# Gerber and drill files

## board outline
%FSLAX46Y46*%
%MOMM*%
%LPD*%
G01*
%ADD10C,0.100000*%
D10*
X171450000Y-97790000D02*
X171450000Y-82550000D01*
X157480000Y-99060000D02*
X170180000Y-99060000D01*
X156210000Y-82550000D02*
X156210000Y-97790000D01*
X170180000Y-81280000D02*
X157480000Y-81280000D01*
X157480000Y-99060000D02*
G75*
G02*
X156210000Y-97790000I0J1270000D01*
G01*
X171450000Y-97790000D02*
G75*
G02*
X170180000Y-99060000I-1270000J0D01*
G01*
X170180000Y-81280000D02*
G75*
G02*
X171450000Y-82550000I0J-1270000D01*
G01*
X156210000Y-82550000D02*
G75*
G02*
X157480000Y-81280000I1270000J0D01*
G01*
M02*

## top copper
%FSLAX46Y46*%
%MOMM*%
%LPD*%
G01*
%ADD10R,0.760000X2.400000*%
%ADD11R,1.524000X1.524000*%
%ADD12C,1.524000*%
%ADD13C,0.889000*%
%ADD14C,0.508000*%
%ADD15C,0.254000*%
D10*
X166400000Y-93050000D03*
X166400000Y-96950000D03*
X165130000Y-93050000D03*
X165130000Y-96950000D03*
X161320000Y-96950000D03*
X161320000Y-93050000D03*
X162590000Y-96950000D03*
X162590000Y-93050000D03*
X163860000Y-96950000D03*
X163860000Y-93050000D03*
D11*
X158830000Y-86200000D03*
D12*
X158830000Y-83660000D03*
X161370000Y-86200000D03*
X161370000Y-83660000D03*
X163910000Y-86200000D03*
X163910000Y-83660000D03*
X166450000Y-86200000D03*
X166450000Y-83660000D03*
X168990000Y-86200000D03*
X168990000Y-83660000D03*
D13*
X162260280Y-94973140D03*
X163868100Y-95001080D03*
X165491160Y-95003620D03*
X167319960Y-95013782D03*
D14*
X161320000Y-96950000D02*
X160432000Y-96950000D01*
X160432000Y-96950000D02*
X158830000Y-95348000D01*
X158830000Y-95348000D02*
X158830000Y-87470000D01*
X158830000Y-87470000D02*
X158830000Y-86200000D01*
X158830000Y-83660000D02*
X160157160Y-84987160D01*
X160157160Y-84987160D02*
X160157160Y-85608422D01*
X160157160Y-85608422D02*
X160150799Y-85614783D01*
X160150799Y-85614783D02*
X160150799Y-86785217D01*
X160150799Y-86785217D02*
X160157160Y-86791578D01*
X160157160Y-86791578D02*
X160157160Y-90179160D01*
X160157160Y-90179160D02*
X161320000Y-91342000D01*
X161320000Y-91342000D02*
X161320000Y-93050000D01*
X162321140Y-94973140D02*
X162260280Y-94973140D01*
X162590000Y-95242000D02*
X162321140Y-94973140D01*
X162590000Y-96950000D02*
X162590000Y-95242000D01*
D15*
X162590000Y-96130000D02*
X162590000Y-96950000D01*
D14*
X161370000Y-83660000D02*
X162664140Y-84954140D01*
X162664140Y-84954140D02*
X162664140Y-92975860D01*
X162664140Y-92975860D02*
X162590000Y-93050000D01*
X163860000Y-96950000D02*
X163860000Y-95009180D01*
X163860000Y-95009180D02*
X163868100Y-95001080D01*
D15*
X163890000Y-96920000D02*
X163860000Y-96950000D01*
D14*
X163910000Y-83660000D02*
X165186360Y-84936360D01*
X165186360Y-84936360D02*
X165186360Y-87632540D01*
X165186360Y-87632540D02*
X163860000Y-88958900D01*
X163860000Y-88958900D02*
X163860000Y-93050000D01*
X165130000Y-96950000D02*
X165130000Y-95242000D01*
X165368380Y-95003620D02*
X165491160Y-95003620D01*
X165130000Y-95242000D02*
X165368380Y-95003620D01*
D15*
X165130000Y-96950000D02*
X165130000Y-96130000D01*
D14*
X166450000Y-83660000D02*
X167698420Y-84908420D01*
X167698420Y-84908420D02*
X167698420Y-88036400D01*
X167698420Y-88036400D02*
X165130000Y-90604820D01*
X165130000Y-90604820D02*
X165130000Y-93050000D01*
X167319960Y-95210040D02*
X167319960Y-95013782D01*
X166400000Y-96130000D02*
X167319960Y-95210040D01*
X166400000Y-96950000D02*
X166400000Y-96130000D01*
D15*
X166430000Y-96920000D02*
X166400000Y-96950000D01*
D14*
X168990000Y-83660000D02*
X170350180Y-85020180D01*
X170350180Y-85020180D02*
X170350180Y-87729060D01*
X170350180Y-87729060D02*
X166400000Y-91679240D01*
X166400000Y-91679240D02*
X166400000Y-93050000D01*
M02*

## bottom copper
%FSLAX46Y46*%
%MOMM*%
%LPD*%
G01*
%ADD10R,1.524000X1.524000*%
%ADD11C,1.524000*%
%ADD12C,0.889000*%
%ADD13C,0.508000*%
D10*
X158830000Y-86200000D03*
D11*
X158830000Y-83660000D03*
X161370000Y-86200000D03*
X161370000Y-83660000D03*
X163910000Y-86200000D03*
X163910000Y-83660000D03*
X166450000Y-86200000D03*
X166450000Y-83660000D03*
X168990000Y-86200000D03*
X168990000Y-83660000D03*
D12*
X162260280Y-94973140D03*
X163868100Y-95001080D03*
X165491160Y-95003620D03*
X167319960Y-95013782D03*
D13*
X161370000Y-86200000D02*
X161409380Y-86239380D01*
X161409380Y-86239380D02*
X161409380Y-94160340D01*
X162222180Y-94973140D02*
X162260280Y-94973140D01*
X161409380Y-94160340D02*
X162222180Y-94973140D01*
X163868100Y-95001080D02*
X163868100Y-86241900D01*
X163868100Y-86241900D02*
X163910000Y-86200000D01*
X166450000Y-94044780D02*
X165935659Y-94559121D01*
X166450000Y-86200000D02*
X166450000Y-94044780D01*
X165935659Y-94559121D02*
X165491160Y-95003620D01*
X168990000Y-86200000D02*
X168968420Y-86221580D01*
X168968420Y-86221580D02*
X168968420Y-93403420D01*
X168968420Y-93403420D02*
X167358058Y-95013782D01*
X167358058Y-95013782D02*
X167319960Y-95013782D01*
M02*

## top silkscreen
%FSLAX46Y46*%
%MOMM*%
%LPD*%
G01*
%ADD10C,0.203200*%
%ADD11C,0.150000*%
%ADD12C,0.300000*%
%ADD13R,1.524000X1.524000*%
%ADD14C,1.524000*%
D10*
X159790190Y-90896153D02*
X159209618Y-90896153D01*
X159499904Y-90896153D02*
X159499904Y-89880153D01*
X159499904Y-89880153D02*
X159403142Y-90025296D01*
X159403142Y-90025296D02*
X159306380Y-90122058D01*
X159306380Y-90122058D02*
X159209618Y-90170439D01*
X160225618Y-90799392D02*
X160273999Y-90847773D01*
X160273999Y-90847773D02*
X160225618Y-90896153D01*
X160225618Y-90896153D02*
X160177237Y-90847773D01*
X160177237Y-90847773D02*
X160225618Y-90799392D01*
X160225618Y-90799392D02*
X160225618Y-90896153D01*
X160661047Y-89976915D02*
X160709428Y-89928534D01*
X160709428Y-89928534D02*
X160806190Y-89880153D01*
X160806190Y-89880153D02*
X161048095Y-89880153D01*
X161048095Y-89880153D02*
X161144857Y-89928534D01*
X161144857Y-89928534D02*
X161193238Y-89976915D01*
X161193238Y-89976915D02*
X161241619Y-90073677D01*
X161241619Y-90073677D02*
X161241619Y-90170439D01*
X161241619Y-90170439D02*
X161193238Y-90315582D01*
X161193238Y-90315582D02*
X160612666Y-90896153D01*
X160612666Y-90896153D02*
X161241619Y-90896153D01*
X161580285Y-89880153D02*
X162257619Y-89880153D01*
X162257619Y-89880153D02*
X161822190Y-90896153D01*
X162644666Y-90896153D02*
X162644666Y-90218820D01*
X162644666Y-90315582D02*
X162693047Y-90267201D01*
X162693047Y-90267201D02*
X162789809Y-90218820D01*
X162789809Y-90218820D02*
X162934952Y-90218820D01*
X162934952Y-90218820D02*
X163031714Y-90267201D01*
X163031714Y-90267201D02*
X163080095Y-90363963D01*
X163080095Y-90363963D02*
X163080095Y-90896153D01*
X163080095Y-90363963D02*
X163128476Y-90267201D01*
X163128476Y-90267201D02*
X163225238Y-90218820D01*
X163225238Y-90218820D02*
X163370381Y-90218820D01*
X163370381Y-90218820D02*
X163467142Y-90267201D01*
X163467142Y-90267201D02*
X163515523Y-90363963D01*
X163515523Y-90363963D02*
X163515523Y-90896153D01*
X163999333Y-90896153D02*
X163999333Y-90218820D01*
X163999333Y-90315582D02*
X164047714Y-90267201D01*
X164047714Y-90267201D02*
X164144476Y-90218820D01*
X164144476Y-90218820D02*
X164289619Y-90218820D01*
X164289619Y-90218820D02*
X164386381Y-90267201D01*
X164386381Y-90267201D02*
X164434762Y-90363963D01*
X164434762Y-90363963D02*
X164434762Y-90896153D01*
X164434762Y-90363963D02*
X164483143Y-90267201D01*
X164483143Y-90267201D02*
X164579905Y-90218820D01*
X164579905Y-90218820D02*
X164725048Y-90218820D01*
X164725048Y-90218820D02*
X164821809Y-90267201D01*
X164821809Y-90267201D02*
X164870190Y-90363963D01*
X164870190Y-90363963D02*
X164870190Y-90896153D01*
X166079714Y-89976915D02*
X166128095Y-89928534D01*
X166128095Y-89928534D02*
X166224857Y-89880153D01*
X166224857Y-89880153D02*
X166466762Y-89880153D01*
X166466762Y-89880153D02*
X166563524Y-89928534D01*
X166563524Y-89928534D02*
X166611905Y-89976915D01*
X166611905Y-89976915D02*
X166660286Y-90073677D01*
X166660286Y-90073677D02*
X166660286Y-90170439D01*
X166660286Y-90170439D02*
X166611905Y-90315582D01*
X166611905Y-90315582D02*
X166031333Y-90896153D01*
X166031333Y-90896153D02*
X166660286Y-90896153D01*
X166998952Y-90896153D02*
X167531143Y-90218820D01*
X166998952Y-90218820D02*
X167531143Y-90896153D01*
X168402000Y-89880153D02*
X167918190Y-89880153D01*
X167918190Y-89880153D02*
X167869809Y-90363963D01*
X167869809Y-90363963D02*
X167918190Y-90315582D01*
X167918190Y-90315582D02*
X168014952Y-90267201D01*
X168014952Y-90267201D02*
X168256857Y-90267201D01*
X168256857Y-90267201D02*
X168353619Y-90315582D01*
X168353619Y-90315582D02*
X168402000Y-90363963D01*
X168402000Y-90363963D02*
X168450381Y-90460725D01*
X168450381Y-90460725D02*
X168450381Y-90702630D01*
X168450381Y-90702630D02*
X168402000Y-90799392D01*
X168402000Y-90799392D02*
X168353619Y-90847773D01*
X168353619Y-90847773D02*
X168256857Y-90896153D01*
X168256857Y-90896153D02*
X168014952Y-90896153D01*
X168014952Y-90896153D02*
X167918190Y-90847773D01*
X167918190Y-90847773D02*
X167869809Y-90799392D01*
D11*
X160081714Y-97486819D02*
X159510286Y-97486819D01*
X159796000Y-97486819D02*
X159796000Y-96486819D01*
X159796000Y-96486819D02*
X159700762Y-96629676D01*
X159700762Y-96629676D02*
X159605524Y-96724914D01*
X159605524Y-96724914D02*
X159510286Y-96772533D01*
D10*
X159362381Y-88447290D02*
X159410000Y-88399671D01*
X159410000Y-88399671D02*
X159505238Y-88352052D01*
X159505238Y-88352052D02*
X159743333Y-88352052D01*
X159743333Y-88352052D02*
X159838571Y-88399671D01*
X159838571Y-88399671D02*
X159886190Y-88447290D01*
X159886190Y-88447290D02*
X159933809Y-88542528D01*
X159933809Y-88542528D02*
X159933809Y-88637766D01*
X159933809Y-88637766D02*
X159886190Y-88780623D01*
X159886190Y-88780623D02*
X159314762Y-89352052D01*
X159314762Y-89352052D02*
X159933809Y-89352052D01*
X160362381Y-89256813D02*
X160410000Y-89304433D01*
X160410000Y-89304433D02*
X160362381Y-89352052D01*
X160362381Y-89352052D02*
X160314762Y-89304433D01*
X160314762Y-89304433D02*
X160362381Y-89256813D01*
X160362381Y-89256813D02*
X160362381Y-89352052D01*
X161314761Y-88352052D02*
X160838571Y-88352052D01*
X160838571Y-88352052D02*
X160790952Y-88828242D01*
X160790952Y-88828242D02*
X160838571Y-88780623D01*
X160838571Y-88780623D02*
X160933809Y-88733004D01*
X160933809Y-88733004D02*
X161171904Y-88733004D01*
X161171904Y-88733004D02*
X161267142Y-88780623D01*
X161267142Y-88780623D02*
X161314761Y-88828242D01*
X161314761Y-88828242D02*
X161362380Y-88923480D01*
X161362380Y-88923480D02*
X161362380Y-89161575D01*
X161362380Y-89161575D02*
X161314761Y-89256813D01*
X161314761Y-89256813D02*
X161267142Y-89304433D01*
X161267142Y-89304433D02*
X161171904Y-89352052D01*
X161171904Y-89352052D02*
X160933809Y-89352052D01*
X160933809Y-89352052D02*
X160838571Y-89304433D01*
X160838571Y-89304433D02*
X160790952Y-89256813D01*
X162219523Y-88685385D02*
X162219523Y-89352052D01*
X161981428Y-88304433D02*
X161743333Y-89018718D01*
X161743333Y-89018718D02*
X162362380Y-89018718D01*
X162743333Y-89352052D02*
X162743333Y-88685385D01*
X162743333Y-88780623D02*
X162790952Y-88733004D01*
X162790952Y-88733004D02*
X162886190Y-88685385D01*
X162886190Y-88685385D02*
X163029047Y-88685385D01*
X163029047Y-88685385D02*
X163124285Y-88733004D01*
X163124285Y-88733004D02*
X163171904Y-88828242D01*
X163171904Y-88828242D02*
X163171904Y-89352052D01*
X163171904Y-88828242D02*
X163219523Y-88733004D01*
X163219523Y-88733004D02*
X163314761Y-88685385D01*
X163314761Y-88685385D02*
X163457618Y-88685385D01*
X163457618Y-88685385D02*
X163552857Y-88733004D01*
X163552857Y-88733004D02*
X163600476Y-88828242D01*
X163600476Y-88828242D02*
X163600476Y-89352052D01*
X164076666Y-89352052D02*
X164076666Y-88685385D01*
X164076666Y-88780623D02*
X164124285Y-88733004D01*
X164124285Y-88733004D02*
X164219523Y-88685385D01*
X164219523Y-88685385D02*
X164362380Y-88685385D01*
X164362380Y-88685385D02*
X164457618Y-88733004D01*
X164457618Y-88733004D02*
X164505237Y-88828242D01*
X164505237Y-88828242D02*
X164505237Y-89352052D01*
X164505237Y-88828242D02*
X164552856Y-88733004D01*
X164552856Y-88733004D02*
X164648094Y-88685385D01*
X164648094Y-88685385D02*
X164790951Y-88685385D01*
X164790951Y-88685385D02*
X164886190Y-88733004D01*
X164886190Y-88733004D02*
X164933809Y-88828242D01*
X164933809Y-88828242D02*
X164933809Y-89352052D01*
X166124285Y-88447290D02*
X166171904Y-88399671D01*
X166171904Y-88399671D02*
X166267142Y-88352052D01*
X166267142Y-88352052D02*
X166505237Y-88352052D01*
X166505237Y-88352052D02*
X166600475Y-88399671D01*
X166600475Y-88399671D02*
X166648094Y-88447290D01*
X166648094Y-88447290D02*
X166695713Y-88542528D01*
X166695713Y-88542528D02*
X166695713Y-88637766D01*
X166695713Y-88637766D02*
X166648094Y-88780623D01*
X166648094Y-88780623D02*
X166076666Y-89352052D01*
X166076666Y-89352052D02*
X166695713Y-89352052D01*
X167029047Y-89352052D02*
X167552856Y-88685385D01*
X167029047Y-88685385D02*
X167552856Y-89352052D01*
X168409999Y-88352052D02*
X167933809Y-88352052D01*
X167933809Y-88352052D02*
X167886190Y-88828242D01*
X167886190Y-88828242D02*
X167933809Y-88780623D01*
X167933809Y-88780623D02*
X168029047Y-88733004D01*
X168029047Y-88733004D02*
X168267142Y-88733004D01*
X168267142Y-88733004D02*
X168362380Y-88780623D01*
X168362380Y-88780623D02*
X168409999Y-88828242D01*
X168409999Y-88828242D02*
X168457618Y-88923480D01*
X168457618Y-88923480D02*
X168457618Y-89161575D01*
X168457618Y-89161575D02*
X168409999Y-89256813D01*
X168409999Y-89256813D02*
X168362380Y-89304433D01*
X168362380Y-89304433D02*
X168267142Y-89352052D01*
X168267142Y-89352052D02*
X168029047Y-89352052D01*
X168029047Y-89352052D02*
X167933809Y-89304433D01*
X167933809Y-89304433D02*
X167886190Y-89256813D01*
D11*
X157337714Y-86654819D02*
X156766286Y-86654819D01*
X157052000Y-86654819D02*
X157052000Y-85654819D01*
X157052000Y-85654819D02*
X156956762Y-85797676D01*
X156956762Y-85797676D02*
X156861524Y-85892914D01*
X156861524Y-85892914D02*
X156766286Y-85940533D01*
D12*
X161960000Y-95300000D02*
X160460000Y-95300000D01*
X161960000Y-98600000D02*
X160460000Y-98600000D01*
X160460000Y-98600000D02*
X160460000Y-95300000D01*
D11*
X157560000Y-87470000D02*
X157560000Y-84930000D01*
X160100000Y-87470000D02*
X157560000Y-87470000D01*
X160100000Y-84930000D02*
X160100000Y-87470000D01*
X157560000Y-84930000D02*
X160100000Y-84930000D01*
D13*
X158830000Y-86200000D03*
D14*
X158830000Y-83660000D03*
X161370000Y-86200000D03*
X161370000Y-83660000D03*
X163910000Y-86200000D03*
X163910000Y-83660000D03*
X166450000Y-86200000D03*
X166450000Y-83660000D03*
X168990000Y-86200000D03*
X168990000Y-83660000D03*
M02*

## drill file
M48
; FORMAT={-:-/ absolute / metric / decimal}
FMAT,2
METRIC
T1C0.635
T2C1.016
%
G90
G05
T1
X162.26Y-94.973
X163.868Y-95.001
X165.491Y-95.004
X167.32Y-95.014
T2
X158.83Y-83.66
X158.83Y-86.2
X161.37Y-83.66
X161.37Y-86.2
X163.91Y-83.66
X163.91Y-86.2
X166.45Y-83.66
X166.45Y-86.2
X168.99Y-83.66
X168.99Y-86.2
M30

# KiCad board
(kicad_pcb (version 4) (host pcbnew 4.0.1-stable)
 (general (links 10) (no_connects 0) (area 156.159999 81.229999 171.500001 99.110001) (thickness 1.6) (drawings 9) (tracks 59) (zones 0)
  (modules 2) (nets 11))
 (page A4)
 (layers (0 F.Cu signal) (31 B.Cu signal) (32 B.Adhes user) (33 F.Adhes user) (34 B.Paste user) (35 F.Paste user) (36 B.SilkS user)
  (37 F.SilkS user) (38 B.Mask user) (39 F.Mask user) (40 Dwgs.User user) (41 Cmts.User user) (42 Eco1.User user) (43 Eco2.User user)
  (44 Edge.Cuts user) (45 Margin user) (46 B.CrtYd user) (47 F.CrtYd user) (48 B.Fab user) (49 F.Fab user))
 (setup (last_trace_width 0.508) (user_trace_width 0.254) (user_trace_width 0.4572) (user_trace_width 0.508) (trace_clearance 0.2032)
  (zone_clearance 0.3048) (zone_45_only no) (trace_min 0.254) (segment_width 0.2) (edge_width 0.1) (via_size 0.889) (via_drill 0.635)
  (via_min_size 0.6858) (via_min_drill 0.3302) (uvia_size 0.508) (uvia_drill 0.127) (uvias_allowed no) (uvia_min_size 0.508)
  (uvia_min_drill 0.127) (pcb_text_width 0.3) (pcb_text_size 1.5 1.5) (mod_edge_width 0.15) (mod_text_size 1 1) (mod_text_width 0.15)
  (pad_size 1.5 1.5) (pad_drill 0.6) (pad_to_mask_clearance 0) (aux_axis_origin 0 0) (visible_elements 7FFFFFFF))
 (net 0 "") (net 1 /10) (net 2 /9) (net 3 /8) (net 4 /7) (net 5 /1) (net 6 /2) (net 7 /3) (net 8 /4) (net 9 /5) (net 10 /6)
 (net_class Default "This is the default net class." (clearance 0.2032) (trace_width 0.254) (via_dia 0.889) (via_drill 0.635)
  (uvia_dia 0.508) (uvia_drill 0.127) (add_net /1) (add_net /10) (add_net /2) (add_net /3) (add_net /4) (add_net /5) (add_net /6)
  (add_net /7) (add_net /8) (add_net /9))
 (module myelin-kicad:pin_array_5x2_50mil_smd (layer F.Cu) (at 163.86 95)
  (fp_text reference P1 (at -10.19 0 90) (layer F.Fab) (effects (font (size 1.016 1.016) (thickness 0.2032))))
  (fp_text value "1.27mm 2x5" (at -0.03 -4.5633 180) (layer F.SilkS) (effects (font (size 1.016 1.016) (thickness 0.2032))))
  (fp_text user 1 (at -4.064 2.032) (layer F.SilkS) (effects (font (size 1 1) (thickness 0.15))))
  (fp_line (start -1.9 0.3) (end -3.4 0.3) (layer F.SilkS) (width 0.3))
  (fp_line (start -1.9 3.6) (end -3.4 3.6) (layer F.SilkS) (width 0.3))
  (fp_line (start -3.4 3.6) (end -3.4 0.3) (layer F.SilkS) (width 0.3))
  (pad 10 smd rect (at 2.54 -1.95) (size 0.76 2.4) (layers F.Cu F.Paste F.Mask) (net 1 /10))
  (pad 9 smd rect (at 2.54 1.95) (size 0.76 2.4) (layers F.Cu F.Paste F.Mask) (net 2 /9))
  (pad 8 smd rect (at 1.27 -1.95) (size 0.76 2.4) (layers F.Cu F.Paste F.Mask) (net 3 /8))
  (pad 7 smd rect (at 1.27 1.95) (size 0.76 2.4) (layers F.Cu F.Paste F.Mask) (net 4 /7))
  (pad 1 smd rect (at -2.54 1.95) (size 0.76 2.4) (layers F.Cu F.Paste F.Mask) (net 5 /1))
  (pad 2 smd rect (at -2.54 -1.95) (size 0.76 2.4) (layers F.Cu F.Paste F.Mask) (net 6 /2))
  (pad 3 smd rect (at -1.27 1.95) (size 0.76 2.4) (layers F.Cu F.Paste F.Mask) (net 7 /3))
  (pad 4 smd rect (at -1.27 -1.95) (size 0.76 2.4) (layers F.Cu F.Paste F.Mask) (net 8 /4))
  (pad 5 smd rect (at 0 1.95) (size 0.76 2.4) (layers F.Cu F.Paste F.Mask) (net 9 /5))
  (pad 6 smd rect (at 0 -1.95) (size 0.76 2.4) (layers F.Cu F.Paste F.Mask) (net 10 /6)))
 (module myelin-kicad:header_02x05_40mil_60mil (layer F.Cu) (at 163.91 84.93)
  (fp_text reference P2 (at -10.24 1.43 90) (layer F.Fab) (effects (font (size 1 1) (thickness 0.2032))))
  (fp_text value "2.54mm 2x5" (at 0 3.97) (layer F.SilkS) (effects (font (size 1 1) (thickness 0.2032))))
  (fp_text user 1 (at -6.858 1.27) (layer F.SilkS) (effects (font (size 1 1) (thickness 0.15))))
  (fp_line (start -6.35 2.54) (end -6.35 0) (layer F.SilkS) (width 0.15))
  (fp_line (start -3.81 2.54) (end -6.35 2.54) (layer F.SilkS) (width 0.15))
  (fp_line (start -3.81 0) (end -3.81 2.54) (layer F.SilkS) (width 0.15))
  (fp_line (start -6.35 0) (end -3.81 0) (layer F.SilkS) (width 0.15))
  (pad 1 thru_hole rect (at -5.08 1.27) (size 1.524 1.524) (drill 1.016) (layers *.Cu *.Mask F.SilkS) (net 5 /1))
  (pad 2 thru_hole circle (at -5.08 -1.27) (size 1.524 1.524) (drill 1.016) (layers *.Cu *.Mask F.SilkS) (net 6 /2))
  (pad 3 thru_hole circle (at -2.54 1.27) (size 1.524 1.524) (drill 1.016) (layers *.Cu *.Mask F.SilkS) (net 7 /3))
  (pad 4 thru_hole circle (at -2.54 -1.27) (size 1.524 1.524) (drill 1.016) (layers *.Cu *.Mask F.SilkS) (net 8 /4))
  (pad 5 thru_hole circle (at 0 1.27) (size 1.524 1.524) (drill 1.016) (layers *.Cu *.Mask F.SilkS) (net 9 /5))
  (pad 6 thru_hole circle (at 0 -1.27) (size 1.524 1.524) (drill 1.016) (layers *.Cu *.Mask F.SilkS) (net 10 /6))
  (pad 7 thru_hole circle (at 2.54 1.27) (size 1.524 1.524) (drill 1.016) (layers *.Cu *.Mask F.SilkS) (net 4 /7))
  (pad 8 thru_hole circle (at 2.54 -1.27) (size 1.524 1.524) (drill 1.016) (layers *.Cu *.Mask F.SilkS) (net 3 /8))
  (pad 9 thru_hole circle (at 5.08 1.27) (size 1.524 1.524) (drill 1.016) (layers *.Cu *.Mask F.SilkS) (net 2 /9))
  (pad 10 thru_hole circle (at 5.08 -1.27) (size 1.524 1.524) (drill 1.016) (layers *.Cu *.Mask F.SilkS) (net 1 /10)))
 (gr_line (start 171.45 97.79) (end 171.45 82.55) (layer Edge.Cuts) (width 0.1))
 (gr_line (start 157.48 99.06) (end 170.18 99.06) (layer Edge.Cuts) (width 0.1))
 (gr_line (start 156.21 82.55) (end 156.21 97.79) (layer Edge.Cuts) (width 0.1))
 (gr_line (start 170.18 81.28) (end 157.48 81.28) (layer Edge.Cuts) (width 0.1))
 (gr_arc (start 157.48 97.79) (end 157.48 99.06) (angle 90) (layer Edge.Cuts) (width 0.1))
 (gr_arc (start 170.18 97.79) (end 171.45 97.79) (angle 90) (layer Edge.Cuts) (width 0.1))
 (gr_arc (start 170.18 82.55) (end 170.18 81.28) (angle 90) (layer Edge.Cuts) (width 0.1))
 (gr_arc (start 157.48 82.55) (end 156.21 82.55) (angle 90) (layer Edge.Cuts) (width 0.1))
 (segment (start 161.32 96.95) (end 160.432 96.95) (width 0.508) (layer F.Cu) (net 5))
 (segment (start 160.432 96.95) (end 158.83 95.348) (width 0.508) (layer F.Cu) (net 5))
 (segment (start 158.83 95.348) (end 158.83 87.47) (width 0.508) (layer F.Cu) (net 5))
 (segment (start 158.83 87.47) (end 158.83 86.2) (width 0.508) (layer F.Cu) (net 5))
 (segment (start 158.83 83.66) (end 160.15716 84.98716) (width 0.508) (layer F.Cu) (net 6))
 (segment (start 160.15716 84.98716) (end 160.15716 85.608422) (width 0.508) (layer F.Cu) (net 6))
 (segment (start 160.15716 85.608422) (end 160.150799 85.614783) (width 0.508) (layer F.Cu) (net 6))
 (segment (start 160.150799 85.614783) (end 160.150799 86.785217) (width 0.508) (layer F.Cu) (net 6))
 (segment (start 160.150799 86.785217) (end 160.15716 86.791578) (width 0.508) (layer F.Cu) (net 6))
 (segment (start 160.15716 86.791578) (end 160.15716 90.17916) (width 0.508) (layer F.Cu) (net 6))
 (segment (start 160.15716 90.17916) (end 161.32 91.342) (width 0.508) (layer F.Cu) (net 6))
 (segment (start 161.32 91.342) (end 161.32 93.05) (width 0.508) (layer F.Cu) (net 6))
 (segment (start 161.37 86.2) (end 161.40938 86.23938) (width 0.508) (layer B.Cu) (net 7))
 (segment (start 161.40938 86.23938) (end 161.40938 94.16034) (width 0.508) (layer B.Cu) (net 7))
 (segment (start 162.22218 94.97314) (end 162.26028 94.97314) (width 0.508) (layer B.Cu) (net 7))
 (segment (start 161.40938 94.16034) (end 162.22218 94.97314) (width 0.508) (layer B.Cu) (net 7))
 (segment (start 162.32114 94.97314) (end 162.26028 94.97314) (width 0.508) (layer F.Cu) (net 7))
 (segment (start 162.59 95.242) (end 162.32114 94.97314) (width 0.508) (layer F.Cu) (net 7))
 (segment (start 162.59 96.95) (end 162.59 95.242) (width 0.508) (layer F.Cu) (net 7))
 (segment (start 162.59 96.13) (end 162.59 96.95) (width 0.254) (layer F.Cu) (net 7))
 (segment (start 161.37 83.66) (end 162.66414 84.95414) (width 0.508) (layer F.Cu) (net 8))
 (segment (start 162.66414 84.95414) (end 162.66414 92.97586) (width 0.508) (layer F.Cu) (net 8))
 (segment (start 162.66414 92.97586) (end 162.59 93.05) (width 0.508) (layer F.Cu) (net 8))
 (segment (start 163.8681 95.00108) (end 163.8681 86.2419) (width 0.508) (layer B.Cu) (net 9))
 (segment (start 163.8681 86.2419) (end 163.91 86.2) (width 0.508) (layer B.Cu) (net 9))
 (segment (start 163.86 96.95) (end 163.86 95.00918) (width 0.508) (layer F.Cu) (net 9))
 (segment (start 163.86 95.00918) (end 163.8681 95.00108) (width 0.508) (layer F.Cu) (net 9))
 (segment (start 163.89 96.92) (end 163.86 96.95) (width 0.254) (layer F.Cu) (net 9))
 (segment (start 163.91 83.66) (end 165.18636 84.93636) (width 0.508) (layer F.Cu) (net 10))
 (segment (start 165.18636 84.93636) (end 165.18636 87.63254) (width 0.508) (layer F.Cu) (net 10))
 (segment (start 165.18636 87.63254) (end 163.86 88.9589) (width 0.508) (layer F.Cu) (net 10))
 (segment (start 163.86 88.9589) (end 163.86 93.05) (width 0.508) (layer F.Cu) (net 10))
 (segment (start 165.13 96.95) (end 165.13 95.242) (width 0.508) (layer F.Cu) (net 4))
 (segment (start 166.45 94.04478) (end 165.935659 94.559121) (width 0.508) (layer B.Cu) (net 4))
 (segment (start 165.36838 95.00362) (end 165.49116 95.00362) (width 0.508) (layer F.Cu) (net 4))
 (segment (start 166.45 86.2) (end 166.45 94.04478) (width 0.508) (layer B.Cu) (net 4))
 (segment (start 165.13 95.242) (end 165.36838 95.00362) (width 0.508) (layer F.Cu) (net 4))
 (segment (start 165.935659 94.559121) (end 165.49116 95.00362) (width 0.508) (layer B.Cu) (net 4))
 (segment (start 165.13 96.95) (end 165.13 96.13) (width 0.254) (layer F.Cu) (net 4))
 (segment (start 166.45 83.66) (end 167.69842 84.90842) (width 0.508) (layer F.Cu) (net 3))
 (segment (start 167.69842 84.90842) (end 167.69842 88.0364) (width 0.508) (layer F.Cu) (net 3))
 (segment (start 167.69842 88.0364) (end 165.13 90.60482) (width 0.508) (layer F.Cu) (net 3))
 (segment (start 165.13 90.60482) (end 165.13 93.05) (width 0.508) (layer F.Cu) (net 3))
 (segment (start 168.99 86.2) (end 168.96842 86.22158) (width 0.508) (layer B.Cu) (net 2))
 (segment (start 168.96842 86.22158) (end 168.96842 93.40342) (width 0.508) (layer B.Cu) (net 2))
 (segment (start 168.96842 93.40342) (end 167.358058 95.013782) (width 0.508) (layer B.Cu) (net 2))
 (segment (start 167.358058 95.013782) (end 167.31996 95.013782) (width 0.508) (layer B.Cu) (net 2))
 (segment (start 167.31996 95.21004) (end 167.31996 95.013782) (width 0.508) (layer F.Cu) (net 2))
 (segment (start 166.4 96.13) (end 167.31996 95.21004) (width 0.508) (layer F.Cu) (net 2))
 (segment (start 166.4 96.95) (end 166.4 96.13) (width 0.508) (layer F.Cu) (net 2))
 (segment (start 166.43 96.92) (end 166.4 96.95) (width 0.254) (layer F.Cu) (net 2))
 (segment (start 168.99 83.66) (end 170.35018 85.02018) (width 0.508) (layer F.Cu) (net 1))
 (segment (start 170.35018 85.02018) (end 170.35018 87.72906) (width 0.508) (layer F.Cu) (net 1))
 (segment (start 170.35018 87.72906) (end 166.4 91.67924) (width 0.508) (layer F.Cu) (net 1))
 (segment (start 166.4 91.67924) (end 166.4 93.05) (width 0.508) (layer F.Cu) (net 1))
 (via (at 162.26028 94.97314) (size 0.889) (drill 0.635) (layers F.Cu B.Cu) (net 7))
 (via (at 163.8681 95.00108) (size 0.889) (drill 0.635) (layers F.Cu B.Cu) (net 9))
 (via (at 165.49116 95.00362) (size 0.889) (drill 0.635) (layers F.Cu B.Cu) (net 4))
 (via (at 167.31996 95.013782) (size 0.889) (drill 0.635) (layers F.Cu B.Cu) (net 2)))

